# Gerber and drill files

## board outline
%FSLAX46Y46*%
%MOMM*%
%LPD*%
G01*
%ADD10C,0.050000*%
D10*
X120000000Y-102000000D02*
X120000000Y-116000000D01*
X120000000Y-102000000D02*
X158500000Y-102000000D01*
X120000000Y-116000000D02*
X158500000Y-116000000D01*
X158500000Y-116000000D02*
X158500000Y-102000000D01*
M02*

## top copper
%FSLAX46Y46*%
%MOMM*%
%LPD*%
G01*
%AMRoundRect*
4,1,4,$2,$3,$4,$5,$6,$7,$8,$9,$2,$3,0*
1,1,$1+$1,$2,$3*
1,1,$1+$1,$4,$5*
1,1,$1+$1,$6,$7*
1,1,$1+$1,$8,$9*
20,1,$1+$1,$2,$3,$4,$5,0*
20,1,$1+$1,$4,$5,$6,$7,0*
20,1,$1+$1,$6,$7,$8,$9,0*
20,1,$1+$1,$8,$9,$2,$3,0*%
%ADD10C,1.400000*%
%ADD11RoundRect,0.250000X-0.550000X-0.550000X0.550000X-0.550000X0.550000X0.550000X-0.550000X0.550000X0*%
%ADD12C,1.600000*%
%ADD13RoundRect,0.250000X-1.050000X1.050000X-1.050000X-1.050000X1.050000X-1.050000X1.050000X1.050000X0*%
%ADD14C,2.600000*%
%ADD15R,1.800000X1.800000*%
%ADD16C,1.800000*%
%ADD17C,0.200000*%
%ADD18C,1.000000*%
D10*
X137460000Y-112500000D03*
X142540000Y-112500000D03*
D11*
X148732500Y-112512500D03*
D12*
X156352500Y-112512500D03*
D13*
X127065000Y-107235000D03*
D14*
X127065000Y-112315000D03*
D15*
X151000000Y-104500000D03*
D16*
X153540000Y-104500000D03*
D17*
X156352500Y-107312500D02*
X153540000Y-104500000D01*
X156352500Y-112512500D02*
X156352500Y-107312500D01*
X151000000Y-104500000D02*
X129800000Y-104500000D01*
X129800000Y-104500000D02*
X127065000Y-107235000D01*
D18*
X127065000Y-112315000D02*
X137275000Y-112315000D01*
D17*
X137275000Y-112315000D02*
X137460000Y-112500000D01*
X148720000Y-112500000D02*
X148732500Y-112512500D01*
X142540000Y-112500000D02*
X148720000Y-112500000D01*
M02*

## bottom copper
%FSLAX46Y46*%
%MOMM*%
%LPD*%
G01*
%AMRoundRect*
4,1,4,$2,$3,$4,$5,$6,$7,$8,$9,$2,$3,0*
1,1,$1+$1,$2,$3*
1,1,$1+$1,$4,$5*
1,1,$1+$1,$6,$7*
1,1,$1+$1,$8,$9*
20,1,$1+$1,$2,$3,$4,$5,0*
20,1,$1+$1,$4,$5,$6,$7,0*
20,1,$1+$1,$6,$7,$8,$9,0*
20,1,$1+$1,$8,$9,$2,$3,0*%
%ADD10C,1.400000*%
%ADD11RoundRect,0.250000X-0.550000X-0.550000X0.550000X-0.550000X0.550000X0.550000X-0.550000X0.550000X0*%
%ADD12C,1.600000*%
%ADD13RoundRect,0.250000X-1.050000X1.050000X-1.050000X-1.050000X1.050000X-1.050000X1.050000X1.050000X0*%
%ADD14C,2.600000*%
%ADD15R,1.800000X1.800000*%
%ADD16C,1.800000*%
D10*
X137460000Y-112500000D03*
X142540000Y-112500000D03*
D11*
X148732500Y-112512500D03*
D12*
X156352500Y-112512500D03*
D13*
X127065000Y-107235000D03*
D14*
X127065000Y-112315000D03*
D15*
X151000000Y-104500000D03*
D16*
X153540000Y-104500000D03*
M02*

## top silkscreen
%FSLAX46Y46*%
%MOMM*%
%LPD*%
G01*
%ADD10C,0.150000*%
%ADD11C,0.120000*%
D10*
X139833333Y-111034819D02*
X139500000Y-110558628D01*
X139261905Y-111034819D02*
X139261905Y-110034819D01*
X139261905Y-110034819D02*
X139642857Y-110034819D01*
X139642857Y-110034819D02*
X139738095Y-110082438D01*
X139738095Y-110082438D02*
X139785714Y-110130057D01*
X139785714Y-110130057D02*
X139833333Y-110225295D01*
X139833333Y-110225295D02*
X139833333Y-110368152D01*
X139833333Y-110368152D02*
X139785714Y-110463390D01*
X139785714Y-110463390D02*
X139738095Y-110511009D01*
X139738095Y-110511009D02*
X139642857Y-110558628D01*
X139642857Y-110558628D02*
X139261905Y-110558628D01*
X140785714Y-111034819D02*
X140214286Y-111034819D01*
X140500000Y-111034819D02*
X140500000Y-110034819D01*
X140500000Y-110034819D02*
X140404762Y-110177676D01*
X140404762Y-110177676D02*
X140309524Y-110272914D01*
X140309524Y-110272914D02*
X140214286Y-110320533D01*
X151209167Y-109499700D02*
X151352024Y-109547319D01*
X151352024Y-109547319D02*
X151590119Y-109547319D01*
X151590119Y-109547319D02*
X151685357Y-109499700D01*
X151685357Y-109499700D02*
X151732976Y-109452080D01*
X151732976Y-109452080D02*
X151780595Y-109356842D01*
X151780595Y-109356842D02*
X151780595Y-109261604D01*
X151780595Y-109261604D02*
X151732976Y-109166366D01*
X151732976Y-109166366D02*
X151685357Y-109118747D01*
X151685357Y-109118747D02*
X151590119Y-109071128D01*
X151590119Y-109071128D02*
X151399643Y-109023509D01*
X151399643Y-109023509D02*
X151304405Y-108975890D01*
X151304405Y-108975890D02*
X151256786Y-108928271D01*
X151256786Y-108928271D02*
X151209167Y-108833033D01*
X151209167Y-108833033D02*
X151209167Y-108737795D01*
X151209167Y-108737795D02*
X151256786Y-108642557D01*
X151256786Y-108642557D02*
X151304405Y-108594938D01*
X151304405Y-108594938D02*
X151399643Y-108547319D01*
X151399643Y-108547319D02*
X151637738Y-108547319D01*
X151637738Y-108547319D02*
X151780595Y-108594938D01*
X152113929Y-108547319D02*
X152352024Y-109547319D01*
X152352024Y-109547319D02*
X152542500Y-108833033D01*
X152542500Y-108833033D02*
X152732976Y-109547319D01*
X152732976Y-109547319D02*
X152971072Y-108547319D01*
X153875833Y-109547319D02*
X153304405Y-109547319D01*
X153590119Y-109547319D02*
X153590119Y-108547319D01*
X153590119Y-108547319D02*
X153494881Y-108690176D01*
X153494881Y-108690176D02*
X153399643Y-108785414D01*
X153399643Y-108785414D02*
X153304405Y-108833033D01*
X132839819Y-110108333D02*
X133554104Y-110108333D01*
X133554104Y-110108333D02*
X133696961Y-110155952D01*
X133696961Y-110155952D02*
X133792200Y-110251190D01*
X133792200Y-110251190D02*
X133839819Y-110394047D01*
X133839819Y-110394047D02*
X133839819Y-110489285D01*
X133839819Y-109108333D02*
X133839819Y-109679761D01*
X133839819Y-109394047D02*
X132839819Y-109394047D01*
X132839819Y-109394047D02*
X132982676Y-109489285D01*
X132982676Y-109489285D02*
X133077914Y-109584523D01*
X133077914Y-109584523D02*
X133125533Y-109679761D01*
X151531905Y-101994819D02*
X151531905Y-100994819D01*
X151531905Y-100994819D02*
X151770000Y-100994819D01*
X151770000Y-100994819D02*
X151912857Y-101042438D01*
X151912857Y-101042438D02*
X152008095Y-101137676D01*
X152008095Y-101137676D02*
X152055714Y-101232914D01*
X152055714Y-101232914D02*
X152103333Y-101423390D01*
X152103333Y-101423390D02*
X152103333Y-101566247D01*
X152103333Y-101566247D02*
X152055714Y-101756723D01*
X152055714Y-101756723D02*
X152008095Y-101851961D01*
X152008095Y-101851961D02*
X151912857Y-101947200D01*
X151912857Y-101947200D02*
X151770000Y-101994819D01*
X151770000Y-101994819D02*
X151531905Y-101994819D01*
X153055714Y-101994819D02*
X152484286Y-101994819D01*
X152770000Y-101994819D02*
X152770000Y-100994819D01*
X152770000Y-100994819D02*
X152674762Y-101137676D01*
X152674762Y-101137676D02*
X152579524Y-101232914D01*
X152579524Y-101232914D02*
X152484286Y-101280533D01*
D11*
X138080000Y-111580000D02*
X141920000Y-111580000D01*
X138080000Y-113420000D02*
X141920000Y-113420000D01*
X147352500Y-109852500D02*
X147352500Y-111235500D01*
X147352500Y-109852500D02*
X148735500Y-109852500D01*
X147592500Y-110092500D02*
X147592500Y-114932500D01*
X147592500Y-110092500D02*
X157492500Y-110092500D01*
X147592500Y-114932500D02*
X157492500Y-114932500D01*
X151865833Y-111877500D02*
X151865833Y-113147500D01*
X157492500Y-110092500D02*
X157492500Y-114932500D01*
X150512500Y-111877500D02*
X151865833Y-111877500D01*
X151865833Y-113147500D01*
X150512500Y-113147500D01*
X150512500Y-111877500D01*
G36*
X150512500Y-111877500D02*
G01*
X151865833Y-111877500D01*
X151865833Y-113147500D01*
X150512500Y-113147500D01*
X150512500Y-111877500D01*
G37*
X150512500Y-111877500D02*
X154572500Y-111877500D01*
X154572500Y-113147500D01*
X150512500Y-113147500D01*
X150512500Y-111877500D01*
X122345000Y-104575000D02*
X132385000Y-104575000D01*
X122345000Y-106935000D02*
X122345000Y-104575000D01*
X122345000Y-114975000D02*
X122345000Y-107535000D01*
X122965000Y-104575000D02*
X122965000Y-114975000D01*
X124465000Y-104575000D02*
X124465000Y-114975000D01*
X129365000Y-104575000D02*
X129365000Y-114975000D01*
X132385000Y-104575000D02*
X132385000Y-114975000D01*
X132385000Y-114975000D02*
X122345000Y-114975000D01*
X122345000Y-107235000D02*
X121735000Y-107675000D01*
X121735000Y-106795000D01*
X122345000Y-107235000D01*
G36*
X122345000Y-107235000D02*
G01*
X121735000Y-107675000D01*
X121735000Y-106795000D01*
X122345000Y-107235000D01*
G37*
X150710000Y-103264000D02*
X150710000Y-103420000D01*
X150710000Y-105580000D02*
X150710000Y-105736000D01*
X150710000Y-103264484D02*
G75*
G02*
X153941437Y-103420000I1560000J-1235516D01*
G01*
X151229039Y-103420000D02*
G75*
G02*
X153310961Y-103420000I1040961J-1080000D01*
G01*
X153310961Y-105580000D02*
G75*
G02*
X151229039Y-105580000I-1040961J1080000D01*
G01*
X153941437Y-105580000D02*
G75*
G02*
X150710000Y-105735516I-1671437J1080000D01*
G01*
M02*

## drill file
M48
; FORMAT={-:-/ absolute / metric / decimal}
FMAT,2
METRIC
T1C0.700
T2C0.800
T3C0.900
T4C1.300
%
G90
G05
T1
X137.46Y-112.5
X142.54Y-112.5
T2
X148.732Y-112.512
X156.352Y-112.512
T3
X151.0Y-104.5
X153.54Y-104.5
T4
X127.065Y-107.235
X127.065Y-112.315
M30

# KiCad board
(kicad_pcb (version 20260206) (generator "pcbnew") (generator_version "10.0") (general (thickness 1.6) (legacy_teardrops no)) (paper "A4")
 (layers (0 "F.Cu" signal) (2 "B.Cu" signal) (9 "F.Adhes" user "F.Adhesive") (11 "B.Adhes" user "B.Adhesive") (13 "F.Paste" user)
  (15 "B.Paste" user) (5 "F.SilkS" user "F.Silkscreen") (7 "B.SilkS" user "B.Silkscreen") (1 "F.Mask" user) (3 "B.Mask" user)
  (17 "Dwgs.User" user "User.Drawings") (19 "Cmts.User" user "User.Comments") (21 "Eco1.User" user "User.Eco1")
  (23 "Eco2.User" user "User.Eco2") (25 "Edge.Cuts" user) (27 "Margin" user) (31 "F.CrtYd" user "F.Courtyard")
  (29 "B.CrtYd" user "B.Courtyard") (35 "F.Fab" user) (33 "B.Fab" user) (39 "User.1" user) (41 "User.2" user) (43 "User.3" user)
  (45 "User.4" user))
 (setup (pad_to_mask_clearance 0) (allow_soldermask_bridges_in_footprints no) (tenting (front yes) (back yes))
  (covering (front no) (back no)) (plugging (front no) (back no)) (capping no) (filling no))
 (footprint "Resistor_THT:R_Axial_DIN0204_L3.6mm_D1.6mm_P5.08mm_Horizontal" (layer "F.Cu") (at 137.46 112.5)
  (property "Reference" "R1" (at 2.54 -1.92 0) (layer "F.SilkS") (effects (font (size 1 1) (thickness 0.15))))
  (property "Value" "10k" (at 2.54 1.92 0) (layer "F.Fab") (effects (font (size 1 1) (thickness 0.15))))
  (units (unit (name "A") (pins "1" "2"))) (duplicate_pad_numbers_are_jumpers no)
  (fp_line (start 0.62 -0.92) (end 4.46 -0.92) (stroke (width 0.12) (type solid)) (layer "F.SilkS"))
  (fp_line (start 0.62 0.92) (end 4.46 0.92) (stroke (width 0.12) (type solid)) (layer "F.SilkS"))
  (pad "1" thru_hole circle (at 0 0) (size 1.4 1.4) (drill 0.7) (layers "*.Cu" "*.Mask") (remove_unused_layers no) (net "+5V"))
  (pad "2" thru_hole circle (at 5.08 0) (size 1.4 1.4) (drill 0.7) (layers "*.Cu" "*.Mask") (remove_unused_layers no) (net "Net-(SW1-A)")))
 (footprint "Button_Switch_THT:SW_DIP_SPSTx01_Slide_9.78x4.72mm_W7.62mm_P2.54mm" (layer "F.Cu") (at 148.7325 112.5125)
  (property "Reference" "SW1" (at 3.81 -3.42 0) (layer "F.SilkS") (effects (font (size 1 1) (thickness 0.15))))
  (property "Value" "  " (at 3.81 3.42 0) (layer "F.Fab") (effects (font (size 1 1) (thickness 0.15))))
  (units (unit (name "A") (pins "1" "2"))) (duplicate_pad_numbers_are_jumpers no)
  (fp_line (start -1.38 -2.66) (end -1.38 -1.277) (stroke (width 0.12) (type solid)) (layer "F.SilkS"))
  (fp_line (start -1.38 -2.66) (end 0.003 -2.66) (stroke (width 0.12) (type solid)) (layer "F.SilkS"))
  (fp_line (start -1.14 -2.42) (end -1.14 2.42) (stroke (width 0.12) (type solid)) (layer "F.SilkS"))
  (fp_line (start -1.14 -2.42) (end 8.76 -2.42) (stroke (width 0.12) (type solid)) (layer "F.SilkS"))
  (fp_line (start -1.14 2.42) (end 8.76 2.42) (stroke (width 0.12) (type solid)) (layer "F.SilkS"))
  (fp_line (start 3.133333 -0.635) (end 3.133333 0.635) (stroke (width 0.12) (type solid)) (layer "F.SilkS"))
  (fp_line (start 8.76 -2.42) (end 8.76 2.42) (stroke (width 0.12) (type solid)) (layer "F.SilkS"))
  (fp_rect (start 1.78 -0.635) (end 3.133333 0.635) (stroke (width 0.12) (type solid)) (fill yes) (layer "F.SilkS"))
  (fp_rect (start 1.78 -0.635) (end 5.84 0.635) (stroke (width 0.12) (type solid)) (fill no) (layer "F.SilkS"))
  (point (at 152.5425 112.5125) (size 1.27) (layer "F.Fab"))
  (pad "1" thru_hole roundrect (at 0 0) (size 1.6 1.6) (drill 0.8) (layers "*.Cu" "*.Mask") (remove_unused_layers no)
   (roundrect_rratio 0.15625) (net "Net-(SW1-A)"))
  (pad "2" thru_hole circle (at 7.62 0) (size 1.6 1.6) (drill 0.8) (layers "*.Cu" "*.Mask") (remove_unused_layers no) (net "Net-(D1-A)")))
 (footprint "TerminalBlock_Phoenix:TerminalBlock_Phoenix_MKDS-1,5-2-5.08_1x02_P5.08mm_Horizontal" (layer "F.Cu") (at 127.065 107.235 -90)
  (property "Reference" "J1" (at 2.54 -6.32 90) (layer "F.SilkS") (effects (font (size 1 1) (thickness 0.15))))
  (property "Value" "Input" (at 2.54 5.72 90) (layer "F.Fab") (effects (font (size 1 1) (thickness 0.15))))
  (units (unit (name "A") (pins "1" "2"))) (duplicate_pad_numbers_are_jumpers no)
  (fp_line (start -2.66 4.72) (end -2.66 -5.32) (stroke (width 0.12) (type solid)) (layer "F.SilkS"))
  (fp_line (start -0.3 4.72) (end -2.66 4.72) (stroke (width 0.12) (type solid)) (layer "F.SilkS"))
  (fp_line (start 7.74 4.72) (end 0.3 4.72) (stroke (width 0.12) (type solid)) (layer "F.SilkS"))
  (fp_line (start -2.66 4.1) (end 7.74 4.1) (stroke (width 0.12) (type solid)) (layer "F.SilkS"))
  (fp_line (start -2.66 2.6) (end 7.74 2.6) (stroke (width 0.12) (type solid)) (layer "F.SilkS"))
  (fp_line (start -2.66 -2.3) (end 7.74 -2.3) (stroke (width 0.12) (type solid)) (layer "F.SilkS"))
  (fp_line (start -2.66 -5.32) (end 7.74 -5.32) (stroke (width 0.12) (type solid)) (layer "F.SilkS"))
  (fp_line (start 7.74 -5.32) (end 7.74 4.72) (stroke (width 0.12) (type solid)) (layer "F.SilkS"))
  (fp_poly (pts (xy 0 4.72) (xy 0.44 5.33) (xy -0.44 5.33)) (stroke (width 0.12) (type solid)) (fill yes) (layer "F.SilkS"))
  (pad "1" thru_hole roundrect (at 0 0 270) (size 2.6 2.6) (drill 1.3) (layers "*.Cu" "*.Mask") (remove_unused_layers no)
   (roundrect_rratio 0.096154) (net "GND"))
  (pad "2" thru_hole circle (at 5.08 0 270) (size 2.6 2.6) (drill 1.3) (layers "*.Cu" "*.Mask") (remove_unused_layers no) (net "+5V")))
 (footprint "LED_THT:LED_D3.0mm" (layer "F.Cu") (at 151 104.5)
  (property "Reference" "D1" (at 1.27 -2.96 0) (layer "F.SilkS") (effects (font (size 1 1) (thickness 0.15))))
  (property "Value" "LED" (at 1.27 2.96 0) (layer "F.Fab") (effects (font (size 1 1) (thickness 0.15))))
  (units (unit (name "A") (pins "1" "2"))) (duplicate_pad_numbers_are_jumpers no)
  (fp_line (start -0.29 -1.236) (end -0.29 -1.08) (stroke (width 0.12) (type solid)) (layer "F.SilkS"))
  (fp_line (start -0.29 1.08) (end -0.29 1.236) (stroke (width 0.12) (type solid)) (layer "F.SilkS"))
  (fp_arc (start -0.29 -1.235516) (mid 1.36566 -1.987699) (end 2.941437 -1.08) (stroke (width 0.12) (type solid)) (layer "F.SilkS"))
  (fp_arc (start 0.229039 -1.08) (mid 1.27 -1.5) (end 2.310961 -1.08) (stroke (width 0.12) (type solid)) (layer "F.SilkS"))
  (fp_arc (start 2.310961 1.08) (mid 1.27 1.5) (end 0.229039 1.08) (stroke (width 0.12) (type solid)) (layer "F.SilkS"))
  (fp_arc (start 2.941437 1.08) (mid 1.36566 1.987699) (end -0.29 1.235516) (stroke (width 0.12) (type solid)) (layer "F.SilkS"))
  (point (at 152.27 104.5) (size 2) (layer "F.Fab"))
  (pad "1" thru_hole rect (at 0 0) (size 1.8 1.8) (drill 0.9) (layers "*.Cu" "*.Mask") (remove_unused_layers no) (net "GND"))
  (pad "2" thru_hole circle (at 2.54 0) (size 1.8 1.8) (drill 0.9) (layers "*.Cu" "*.Mask") (remove_unused_layers no) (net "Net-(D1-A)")))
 (gr_line (start 120 102) (end 120 116) (stroke (width 0.05) (type default)) (layer "Edge.Cuts"))
 (gr_line (start 120 102) (end 158.5 102) (stroke (width 0.05) (type default)) (layer "Edge.Cuts"))
 (gr_line (start 120 116) (end 158.5 116) (stroke (width 0.05) (type default)) (layer "Edge.Cuts"))
 (gr_line (start 158.5 116) (end 158.5 102) (stroke (width 0.05) (type default)) (layer "Edge.Cuts"))
 (segment (start 156.3525 107.3125) (end 153.54 104.5) (width 0.2) (layer "F.Cu") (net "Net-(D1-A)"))
 (segment (start 156.3525 112.5125) (end 156.3525 107.3125) (width 0.2) (layer "F.Cu") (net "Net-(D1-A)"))
 (segment (start 151 104.5) (end 129.8 104.5) (width 0.2) (layer "F.Cu") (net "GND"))
 (segment (start 129.8 104.5) (end 127.065 107.235) (width 0.2) (layer "F.Cu") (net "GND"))
 (segment (start 127.065 112.315) (end 137.275 112.315) (width 1) (layer "F.Cu") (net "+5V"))
 (segment (start 137.275 112.315) (end 137.46 112.5) (width 0.2) (layer "F.Cu") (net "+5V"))
 (segment (start 148.72 112.5) (end 148.7325 112.5125) (width 0.2) (layer "F.Cu") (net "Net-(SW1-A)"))
 (segment (start 142.54 112.5) (end 148.72 112.5) (width 0.2) (layer "F.Cu") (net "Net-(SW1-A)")))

